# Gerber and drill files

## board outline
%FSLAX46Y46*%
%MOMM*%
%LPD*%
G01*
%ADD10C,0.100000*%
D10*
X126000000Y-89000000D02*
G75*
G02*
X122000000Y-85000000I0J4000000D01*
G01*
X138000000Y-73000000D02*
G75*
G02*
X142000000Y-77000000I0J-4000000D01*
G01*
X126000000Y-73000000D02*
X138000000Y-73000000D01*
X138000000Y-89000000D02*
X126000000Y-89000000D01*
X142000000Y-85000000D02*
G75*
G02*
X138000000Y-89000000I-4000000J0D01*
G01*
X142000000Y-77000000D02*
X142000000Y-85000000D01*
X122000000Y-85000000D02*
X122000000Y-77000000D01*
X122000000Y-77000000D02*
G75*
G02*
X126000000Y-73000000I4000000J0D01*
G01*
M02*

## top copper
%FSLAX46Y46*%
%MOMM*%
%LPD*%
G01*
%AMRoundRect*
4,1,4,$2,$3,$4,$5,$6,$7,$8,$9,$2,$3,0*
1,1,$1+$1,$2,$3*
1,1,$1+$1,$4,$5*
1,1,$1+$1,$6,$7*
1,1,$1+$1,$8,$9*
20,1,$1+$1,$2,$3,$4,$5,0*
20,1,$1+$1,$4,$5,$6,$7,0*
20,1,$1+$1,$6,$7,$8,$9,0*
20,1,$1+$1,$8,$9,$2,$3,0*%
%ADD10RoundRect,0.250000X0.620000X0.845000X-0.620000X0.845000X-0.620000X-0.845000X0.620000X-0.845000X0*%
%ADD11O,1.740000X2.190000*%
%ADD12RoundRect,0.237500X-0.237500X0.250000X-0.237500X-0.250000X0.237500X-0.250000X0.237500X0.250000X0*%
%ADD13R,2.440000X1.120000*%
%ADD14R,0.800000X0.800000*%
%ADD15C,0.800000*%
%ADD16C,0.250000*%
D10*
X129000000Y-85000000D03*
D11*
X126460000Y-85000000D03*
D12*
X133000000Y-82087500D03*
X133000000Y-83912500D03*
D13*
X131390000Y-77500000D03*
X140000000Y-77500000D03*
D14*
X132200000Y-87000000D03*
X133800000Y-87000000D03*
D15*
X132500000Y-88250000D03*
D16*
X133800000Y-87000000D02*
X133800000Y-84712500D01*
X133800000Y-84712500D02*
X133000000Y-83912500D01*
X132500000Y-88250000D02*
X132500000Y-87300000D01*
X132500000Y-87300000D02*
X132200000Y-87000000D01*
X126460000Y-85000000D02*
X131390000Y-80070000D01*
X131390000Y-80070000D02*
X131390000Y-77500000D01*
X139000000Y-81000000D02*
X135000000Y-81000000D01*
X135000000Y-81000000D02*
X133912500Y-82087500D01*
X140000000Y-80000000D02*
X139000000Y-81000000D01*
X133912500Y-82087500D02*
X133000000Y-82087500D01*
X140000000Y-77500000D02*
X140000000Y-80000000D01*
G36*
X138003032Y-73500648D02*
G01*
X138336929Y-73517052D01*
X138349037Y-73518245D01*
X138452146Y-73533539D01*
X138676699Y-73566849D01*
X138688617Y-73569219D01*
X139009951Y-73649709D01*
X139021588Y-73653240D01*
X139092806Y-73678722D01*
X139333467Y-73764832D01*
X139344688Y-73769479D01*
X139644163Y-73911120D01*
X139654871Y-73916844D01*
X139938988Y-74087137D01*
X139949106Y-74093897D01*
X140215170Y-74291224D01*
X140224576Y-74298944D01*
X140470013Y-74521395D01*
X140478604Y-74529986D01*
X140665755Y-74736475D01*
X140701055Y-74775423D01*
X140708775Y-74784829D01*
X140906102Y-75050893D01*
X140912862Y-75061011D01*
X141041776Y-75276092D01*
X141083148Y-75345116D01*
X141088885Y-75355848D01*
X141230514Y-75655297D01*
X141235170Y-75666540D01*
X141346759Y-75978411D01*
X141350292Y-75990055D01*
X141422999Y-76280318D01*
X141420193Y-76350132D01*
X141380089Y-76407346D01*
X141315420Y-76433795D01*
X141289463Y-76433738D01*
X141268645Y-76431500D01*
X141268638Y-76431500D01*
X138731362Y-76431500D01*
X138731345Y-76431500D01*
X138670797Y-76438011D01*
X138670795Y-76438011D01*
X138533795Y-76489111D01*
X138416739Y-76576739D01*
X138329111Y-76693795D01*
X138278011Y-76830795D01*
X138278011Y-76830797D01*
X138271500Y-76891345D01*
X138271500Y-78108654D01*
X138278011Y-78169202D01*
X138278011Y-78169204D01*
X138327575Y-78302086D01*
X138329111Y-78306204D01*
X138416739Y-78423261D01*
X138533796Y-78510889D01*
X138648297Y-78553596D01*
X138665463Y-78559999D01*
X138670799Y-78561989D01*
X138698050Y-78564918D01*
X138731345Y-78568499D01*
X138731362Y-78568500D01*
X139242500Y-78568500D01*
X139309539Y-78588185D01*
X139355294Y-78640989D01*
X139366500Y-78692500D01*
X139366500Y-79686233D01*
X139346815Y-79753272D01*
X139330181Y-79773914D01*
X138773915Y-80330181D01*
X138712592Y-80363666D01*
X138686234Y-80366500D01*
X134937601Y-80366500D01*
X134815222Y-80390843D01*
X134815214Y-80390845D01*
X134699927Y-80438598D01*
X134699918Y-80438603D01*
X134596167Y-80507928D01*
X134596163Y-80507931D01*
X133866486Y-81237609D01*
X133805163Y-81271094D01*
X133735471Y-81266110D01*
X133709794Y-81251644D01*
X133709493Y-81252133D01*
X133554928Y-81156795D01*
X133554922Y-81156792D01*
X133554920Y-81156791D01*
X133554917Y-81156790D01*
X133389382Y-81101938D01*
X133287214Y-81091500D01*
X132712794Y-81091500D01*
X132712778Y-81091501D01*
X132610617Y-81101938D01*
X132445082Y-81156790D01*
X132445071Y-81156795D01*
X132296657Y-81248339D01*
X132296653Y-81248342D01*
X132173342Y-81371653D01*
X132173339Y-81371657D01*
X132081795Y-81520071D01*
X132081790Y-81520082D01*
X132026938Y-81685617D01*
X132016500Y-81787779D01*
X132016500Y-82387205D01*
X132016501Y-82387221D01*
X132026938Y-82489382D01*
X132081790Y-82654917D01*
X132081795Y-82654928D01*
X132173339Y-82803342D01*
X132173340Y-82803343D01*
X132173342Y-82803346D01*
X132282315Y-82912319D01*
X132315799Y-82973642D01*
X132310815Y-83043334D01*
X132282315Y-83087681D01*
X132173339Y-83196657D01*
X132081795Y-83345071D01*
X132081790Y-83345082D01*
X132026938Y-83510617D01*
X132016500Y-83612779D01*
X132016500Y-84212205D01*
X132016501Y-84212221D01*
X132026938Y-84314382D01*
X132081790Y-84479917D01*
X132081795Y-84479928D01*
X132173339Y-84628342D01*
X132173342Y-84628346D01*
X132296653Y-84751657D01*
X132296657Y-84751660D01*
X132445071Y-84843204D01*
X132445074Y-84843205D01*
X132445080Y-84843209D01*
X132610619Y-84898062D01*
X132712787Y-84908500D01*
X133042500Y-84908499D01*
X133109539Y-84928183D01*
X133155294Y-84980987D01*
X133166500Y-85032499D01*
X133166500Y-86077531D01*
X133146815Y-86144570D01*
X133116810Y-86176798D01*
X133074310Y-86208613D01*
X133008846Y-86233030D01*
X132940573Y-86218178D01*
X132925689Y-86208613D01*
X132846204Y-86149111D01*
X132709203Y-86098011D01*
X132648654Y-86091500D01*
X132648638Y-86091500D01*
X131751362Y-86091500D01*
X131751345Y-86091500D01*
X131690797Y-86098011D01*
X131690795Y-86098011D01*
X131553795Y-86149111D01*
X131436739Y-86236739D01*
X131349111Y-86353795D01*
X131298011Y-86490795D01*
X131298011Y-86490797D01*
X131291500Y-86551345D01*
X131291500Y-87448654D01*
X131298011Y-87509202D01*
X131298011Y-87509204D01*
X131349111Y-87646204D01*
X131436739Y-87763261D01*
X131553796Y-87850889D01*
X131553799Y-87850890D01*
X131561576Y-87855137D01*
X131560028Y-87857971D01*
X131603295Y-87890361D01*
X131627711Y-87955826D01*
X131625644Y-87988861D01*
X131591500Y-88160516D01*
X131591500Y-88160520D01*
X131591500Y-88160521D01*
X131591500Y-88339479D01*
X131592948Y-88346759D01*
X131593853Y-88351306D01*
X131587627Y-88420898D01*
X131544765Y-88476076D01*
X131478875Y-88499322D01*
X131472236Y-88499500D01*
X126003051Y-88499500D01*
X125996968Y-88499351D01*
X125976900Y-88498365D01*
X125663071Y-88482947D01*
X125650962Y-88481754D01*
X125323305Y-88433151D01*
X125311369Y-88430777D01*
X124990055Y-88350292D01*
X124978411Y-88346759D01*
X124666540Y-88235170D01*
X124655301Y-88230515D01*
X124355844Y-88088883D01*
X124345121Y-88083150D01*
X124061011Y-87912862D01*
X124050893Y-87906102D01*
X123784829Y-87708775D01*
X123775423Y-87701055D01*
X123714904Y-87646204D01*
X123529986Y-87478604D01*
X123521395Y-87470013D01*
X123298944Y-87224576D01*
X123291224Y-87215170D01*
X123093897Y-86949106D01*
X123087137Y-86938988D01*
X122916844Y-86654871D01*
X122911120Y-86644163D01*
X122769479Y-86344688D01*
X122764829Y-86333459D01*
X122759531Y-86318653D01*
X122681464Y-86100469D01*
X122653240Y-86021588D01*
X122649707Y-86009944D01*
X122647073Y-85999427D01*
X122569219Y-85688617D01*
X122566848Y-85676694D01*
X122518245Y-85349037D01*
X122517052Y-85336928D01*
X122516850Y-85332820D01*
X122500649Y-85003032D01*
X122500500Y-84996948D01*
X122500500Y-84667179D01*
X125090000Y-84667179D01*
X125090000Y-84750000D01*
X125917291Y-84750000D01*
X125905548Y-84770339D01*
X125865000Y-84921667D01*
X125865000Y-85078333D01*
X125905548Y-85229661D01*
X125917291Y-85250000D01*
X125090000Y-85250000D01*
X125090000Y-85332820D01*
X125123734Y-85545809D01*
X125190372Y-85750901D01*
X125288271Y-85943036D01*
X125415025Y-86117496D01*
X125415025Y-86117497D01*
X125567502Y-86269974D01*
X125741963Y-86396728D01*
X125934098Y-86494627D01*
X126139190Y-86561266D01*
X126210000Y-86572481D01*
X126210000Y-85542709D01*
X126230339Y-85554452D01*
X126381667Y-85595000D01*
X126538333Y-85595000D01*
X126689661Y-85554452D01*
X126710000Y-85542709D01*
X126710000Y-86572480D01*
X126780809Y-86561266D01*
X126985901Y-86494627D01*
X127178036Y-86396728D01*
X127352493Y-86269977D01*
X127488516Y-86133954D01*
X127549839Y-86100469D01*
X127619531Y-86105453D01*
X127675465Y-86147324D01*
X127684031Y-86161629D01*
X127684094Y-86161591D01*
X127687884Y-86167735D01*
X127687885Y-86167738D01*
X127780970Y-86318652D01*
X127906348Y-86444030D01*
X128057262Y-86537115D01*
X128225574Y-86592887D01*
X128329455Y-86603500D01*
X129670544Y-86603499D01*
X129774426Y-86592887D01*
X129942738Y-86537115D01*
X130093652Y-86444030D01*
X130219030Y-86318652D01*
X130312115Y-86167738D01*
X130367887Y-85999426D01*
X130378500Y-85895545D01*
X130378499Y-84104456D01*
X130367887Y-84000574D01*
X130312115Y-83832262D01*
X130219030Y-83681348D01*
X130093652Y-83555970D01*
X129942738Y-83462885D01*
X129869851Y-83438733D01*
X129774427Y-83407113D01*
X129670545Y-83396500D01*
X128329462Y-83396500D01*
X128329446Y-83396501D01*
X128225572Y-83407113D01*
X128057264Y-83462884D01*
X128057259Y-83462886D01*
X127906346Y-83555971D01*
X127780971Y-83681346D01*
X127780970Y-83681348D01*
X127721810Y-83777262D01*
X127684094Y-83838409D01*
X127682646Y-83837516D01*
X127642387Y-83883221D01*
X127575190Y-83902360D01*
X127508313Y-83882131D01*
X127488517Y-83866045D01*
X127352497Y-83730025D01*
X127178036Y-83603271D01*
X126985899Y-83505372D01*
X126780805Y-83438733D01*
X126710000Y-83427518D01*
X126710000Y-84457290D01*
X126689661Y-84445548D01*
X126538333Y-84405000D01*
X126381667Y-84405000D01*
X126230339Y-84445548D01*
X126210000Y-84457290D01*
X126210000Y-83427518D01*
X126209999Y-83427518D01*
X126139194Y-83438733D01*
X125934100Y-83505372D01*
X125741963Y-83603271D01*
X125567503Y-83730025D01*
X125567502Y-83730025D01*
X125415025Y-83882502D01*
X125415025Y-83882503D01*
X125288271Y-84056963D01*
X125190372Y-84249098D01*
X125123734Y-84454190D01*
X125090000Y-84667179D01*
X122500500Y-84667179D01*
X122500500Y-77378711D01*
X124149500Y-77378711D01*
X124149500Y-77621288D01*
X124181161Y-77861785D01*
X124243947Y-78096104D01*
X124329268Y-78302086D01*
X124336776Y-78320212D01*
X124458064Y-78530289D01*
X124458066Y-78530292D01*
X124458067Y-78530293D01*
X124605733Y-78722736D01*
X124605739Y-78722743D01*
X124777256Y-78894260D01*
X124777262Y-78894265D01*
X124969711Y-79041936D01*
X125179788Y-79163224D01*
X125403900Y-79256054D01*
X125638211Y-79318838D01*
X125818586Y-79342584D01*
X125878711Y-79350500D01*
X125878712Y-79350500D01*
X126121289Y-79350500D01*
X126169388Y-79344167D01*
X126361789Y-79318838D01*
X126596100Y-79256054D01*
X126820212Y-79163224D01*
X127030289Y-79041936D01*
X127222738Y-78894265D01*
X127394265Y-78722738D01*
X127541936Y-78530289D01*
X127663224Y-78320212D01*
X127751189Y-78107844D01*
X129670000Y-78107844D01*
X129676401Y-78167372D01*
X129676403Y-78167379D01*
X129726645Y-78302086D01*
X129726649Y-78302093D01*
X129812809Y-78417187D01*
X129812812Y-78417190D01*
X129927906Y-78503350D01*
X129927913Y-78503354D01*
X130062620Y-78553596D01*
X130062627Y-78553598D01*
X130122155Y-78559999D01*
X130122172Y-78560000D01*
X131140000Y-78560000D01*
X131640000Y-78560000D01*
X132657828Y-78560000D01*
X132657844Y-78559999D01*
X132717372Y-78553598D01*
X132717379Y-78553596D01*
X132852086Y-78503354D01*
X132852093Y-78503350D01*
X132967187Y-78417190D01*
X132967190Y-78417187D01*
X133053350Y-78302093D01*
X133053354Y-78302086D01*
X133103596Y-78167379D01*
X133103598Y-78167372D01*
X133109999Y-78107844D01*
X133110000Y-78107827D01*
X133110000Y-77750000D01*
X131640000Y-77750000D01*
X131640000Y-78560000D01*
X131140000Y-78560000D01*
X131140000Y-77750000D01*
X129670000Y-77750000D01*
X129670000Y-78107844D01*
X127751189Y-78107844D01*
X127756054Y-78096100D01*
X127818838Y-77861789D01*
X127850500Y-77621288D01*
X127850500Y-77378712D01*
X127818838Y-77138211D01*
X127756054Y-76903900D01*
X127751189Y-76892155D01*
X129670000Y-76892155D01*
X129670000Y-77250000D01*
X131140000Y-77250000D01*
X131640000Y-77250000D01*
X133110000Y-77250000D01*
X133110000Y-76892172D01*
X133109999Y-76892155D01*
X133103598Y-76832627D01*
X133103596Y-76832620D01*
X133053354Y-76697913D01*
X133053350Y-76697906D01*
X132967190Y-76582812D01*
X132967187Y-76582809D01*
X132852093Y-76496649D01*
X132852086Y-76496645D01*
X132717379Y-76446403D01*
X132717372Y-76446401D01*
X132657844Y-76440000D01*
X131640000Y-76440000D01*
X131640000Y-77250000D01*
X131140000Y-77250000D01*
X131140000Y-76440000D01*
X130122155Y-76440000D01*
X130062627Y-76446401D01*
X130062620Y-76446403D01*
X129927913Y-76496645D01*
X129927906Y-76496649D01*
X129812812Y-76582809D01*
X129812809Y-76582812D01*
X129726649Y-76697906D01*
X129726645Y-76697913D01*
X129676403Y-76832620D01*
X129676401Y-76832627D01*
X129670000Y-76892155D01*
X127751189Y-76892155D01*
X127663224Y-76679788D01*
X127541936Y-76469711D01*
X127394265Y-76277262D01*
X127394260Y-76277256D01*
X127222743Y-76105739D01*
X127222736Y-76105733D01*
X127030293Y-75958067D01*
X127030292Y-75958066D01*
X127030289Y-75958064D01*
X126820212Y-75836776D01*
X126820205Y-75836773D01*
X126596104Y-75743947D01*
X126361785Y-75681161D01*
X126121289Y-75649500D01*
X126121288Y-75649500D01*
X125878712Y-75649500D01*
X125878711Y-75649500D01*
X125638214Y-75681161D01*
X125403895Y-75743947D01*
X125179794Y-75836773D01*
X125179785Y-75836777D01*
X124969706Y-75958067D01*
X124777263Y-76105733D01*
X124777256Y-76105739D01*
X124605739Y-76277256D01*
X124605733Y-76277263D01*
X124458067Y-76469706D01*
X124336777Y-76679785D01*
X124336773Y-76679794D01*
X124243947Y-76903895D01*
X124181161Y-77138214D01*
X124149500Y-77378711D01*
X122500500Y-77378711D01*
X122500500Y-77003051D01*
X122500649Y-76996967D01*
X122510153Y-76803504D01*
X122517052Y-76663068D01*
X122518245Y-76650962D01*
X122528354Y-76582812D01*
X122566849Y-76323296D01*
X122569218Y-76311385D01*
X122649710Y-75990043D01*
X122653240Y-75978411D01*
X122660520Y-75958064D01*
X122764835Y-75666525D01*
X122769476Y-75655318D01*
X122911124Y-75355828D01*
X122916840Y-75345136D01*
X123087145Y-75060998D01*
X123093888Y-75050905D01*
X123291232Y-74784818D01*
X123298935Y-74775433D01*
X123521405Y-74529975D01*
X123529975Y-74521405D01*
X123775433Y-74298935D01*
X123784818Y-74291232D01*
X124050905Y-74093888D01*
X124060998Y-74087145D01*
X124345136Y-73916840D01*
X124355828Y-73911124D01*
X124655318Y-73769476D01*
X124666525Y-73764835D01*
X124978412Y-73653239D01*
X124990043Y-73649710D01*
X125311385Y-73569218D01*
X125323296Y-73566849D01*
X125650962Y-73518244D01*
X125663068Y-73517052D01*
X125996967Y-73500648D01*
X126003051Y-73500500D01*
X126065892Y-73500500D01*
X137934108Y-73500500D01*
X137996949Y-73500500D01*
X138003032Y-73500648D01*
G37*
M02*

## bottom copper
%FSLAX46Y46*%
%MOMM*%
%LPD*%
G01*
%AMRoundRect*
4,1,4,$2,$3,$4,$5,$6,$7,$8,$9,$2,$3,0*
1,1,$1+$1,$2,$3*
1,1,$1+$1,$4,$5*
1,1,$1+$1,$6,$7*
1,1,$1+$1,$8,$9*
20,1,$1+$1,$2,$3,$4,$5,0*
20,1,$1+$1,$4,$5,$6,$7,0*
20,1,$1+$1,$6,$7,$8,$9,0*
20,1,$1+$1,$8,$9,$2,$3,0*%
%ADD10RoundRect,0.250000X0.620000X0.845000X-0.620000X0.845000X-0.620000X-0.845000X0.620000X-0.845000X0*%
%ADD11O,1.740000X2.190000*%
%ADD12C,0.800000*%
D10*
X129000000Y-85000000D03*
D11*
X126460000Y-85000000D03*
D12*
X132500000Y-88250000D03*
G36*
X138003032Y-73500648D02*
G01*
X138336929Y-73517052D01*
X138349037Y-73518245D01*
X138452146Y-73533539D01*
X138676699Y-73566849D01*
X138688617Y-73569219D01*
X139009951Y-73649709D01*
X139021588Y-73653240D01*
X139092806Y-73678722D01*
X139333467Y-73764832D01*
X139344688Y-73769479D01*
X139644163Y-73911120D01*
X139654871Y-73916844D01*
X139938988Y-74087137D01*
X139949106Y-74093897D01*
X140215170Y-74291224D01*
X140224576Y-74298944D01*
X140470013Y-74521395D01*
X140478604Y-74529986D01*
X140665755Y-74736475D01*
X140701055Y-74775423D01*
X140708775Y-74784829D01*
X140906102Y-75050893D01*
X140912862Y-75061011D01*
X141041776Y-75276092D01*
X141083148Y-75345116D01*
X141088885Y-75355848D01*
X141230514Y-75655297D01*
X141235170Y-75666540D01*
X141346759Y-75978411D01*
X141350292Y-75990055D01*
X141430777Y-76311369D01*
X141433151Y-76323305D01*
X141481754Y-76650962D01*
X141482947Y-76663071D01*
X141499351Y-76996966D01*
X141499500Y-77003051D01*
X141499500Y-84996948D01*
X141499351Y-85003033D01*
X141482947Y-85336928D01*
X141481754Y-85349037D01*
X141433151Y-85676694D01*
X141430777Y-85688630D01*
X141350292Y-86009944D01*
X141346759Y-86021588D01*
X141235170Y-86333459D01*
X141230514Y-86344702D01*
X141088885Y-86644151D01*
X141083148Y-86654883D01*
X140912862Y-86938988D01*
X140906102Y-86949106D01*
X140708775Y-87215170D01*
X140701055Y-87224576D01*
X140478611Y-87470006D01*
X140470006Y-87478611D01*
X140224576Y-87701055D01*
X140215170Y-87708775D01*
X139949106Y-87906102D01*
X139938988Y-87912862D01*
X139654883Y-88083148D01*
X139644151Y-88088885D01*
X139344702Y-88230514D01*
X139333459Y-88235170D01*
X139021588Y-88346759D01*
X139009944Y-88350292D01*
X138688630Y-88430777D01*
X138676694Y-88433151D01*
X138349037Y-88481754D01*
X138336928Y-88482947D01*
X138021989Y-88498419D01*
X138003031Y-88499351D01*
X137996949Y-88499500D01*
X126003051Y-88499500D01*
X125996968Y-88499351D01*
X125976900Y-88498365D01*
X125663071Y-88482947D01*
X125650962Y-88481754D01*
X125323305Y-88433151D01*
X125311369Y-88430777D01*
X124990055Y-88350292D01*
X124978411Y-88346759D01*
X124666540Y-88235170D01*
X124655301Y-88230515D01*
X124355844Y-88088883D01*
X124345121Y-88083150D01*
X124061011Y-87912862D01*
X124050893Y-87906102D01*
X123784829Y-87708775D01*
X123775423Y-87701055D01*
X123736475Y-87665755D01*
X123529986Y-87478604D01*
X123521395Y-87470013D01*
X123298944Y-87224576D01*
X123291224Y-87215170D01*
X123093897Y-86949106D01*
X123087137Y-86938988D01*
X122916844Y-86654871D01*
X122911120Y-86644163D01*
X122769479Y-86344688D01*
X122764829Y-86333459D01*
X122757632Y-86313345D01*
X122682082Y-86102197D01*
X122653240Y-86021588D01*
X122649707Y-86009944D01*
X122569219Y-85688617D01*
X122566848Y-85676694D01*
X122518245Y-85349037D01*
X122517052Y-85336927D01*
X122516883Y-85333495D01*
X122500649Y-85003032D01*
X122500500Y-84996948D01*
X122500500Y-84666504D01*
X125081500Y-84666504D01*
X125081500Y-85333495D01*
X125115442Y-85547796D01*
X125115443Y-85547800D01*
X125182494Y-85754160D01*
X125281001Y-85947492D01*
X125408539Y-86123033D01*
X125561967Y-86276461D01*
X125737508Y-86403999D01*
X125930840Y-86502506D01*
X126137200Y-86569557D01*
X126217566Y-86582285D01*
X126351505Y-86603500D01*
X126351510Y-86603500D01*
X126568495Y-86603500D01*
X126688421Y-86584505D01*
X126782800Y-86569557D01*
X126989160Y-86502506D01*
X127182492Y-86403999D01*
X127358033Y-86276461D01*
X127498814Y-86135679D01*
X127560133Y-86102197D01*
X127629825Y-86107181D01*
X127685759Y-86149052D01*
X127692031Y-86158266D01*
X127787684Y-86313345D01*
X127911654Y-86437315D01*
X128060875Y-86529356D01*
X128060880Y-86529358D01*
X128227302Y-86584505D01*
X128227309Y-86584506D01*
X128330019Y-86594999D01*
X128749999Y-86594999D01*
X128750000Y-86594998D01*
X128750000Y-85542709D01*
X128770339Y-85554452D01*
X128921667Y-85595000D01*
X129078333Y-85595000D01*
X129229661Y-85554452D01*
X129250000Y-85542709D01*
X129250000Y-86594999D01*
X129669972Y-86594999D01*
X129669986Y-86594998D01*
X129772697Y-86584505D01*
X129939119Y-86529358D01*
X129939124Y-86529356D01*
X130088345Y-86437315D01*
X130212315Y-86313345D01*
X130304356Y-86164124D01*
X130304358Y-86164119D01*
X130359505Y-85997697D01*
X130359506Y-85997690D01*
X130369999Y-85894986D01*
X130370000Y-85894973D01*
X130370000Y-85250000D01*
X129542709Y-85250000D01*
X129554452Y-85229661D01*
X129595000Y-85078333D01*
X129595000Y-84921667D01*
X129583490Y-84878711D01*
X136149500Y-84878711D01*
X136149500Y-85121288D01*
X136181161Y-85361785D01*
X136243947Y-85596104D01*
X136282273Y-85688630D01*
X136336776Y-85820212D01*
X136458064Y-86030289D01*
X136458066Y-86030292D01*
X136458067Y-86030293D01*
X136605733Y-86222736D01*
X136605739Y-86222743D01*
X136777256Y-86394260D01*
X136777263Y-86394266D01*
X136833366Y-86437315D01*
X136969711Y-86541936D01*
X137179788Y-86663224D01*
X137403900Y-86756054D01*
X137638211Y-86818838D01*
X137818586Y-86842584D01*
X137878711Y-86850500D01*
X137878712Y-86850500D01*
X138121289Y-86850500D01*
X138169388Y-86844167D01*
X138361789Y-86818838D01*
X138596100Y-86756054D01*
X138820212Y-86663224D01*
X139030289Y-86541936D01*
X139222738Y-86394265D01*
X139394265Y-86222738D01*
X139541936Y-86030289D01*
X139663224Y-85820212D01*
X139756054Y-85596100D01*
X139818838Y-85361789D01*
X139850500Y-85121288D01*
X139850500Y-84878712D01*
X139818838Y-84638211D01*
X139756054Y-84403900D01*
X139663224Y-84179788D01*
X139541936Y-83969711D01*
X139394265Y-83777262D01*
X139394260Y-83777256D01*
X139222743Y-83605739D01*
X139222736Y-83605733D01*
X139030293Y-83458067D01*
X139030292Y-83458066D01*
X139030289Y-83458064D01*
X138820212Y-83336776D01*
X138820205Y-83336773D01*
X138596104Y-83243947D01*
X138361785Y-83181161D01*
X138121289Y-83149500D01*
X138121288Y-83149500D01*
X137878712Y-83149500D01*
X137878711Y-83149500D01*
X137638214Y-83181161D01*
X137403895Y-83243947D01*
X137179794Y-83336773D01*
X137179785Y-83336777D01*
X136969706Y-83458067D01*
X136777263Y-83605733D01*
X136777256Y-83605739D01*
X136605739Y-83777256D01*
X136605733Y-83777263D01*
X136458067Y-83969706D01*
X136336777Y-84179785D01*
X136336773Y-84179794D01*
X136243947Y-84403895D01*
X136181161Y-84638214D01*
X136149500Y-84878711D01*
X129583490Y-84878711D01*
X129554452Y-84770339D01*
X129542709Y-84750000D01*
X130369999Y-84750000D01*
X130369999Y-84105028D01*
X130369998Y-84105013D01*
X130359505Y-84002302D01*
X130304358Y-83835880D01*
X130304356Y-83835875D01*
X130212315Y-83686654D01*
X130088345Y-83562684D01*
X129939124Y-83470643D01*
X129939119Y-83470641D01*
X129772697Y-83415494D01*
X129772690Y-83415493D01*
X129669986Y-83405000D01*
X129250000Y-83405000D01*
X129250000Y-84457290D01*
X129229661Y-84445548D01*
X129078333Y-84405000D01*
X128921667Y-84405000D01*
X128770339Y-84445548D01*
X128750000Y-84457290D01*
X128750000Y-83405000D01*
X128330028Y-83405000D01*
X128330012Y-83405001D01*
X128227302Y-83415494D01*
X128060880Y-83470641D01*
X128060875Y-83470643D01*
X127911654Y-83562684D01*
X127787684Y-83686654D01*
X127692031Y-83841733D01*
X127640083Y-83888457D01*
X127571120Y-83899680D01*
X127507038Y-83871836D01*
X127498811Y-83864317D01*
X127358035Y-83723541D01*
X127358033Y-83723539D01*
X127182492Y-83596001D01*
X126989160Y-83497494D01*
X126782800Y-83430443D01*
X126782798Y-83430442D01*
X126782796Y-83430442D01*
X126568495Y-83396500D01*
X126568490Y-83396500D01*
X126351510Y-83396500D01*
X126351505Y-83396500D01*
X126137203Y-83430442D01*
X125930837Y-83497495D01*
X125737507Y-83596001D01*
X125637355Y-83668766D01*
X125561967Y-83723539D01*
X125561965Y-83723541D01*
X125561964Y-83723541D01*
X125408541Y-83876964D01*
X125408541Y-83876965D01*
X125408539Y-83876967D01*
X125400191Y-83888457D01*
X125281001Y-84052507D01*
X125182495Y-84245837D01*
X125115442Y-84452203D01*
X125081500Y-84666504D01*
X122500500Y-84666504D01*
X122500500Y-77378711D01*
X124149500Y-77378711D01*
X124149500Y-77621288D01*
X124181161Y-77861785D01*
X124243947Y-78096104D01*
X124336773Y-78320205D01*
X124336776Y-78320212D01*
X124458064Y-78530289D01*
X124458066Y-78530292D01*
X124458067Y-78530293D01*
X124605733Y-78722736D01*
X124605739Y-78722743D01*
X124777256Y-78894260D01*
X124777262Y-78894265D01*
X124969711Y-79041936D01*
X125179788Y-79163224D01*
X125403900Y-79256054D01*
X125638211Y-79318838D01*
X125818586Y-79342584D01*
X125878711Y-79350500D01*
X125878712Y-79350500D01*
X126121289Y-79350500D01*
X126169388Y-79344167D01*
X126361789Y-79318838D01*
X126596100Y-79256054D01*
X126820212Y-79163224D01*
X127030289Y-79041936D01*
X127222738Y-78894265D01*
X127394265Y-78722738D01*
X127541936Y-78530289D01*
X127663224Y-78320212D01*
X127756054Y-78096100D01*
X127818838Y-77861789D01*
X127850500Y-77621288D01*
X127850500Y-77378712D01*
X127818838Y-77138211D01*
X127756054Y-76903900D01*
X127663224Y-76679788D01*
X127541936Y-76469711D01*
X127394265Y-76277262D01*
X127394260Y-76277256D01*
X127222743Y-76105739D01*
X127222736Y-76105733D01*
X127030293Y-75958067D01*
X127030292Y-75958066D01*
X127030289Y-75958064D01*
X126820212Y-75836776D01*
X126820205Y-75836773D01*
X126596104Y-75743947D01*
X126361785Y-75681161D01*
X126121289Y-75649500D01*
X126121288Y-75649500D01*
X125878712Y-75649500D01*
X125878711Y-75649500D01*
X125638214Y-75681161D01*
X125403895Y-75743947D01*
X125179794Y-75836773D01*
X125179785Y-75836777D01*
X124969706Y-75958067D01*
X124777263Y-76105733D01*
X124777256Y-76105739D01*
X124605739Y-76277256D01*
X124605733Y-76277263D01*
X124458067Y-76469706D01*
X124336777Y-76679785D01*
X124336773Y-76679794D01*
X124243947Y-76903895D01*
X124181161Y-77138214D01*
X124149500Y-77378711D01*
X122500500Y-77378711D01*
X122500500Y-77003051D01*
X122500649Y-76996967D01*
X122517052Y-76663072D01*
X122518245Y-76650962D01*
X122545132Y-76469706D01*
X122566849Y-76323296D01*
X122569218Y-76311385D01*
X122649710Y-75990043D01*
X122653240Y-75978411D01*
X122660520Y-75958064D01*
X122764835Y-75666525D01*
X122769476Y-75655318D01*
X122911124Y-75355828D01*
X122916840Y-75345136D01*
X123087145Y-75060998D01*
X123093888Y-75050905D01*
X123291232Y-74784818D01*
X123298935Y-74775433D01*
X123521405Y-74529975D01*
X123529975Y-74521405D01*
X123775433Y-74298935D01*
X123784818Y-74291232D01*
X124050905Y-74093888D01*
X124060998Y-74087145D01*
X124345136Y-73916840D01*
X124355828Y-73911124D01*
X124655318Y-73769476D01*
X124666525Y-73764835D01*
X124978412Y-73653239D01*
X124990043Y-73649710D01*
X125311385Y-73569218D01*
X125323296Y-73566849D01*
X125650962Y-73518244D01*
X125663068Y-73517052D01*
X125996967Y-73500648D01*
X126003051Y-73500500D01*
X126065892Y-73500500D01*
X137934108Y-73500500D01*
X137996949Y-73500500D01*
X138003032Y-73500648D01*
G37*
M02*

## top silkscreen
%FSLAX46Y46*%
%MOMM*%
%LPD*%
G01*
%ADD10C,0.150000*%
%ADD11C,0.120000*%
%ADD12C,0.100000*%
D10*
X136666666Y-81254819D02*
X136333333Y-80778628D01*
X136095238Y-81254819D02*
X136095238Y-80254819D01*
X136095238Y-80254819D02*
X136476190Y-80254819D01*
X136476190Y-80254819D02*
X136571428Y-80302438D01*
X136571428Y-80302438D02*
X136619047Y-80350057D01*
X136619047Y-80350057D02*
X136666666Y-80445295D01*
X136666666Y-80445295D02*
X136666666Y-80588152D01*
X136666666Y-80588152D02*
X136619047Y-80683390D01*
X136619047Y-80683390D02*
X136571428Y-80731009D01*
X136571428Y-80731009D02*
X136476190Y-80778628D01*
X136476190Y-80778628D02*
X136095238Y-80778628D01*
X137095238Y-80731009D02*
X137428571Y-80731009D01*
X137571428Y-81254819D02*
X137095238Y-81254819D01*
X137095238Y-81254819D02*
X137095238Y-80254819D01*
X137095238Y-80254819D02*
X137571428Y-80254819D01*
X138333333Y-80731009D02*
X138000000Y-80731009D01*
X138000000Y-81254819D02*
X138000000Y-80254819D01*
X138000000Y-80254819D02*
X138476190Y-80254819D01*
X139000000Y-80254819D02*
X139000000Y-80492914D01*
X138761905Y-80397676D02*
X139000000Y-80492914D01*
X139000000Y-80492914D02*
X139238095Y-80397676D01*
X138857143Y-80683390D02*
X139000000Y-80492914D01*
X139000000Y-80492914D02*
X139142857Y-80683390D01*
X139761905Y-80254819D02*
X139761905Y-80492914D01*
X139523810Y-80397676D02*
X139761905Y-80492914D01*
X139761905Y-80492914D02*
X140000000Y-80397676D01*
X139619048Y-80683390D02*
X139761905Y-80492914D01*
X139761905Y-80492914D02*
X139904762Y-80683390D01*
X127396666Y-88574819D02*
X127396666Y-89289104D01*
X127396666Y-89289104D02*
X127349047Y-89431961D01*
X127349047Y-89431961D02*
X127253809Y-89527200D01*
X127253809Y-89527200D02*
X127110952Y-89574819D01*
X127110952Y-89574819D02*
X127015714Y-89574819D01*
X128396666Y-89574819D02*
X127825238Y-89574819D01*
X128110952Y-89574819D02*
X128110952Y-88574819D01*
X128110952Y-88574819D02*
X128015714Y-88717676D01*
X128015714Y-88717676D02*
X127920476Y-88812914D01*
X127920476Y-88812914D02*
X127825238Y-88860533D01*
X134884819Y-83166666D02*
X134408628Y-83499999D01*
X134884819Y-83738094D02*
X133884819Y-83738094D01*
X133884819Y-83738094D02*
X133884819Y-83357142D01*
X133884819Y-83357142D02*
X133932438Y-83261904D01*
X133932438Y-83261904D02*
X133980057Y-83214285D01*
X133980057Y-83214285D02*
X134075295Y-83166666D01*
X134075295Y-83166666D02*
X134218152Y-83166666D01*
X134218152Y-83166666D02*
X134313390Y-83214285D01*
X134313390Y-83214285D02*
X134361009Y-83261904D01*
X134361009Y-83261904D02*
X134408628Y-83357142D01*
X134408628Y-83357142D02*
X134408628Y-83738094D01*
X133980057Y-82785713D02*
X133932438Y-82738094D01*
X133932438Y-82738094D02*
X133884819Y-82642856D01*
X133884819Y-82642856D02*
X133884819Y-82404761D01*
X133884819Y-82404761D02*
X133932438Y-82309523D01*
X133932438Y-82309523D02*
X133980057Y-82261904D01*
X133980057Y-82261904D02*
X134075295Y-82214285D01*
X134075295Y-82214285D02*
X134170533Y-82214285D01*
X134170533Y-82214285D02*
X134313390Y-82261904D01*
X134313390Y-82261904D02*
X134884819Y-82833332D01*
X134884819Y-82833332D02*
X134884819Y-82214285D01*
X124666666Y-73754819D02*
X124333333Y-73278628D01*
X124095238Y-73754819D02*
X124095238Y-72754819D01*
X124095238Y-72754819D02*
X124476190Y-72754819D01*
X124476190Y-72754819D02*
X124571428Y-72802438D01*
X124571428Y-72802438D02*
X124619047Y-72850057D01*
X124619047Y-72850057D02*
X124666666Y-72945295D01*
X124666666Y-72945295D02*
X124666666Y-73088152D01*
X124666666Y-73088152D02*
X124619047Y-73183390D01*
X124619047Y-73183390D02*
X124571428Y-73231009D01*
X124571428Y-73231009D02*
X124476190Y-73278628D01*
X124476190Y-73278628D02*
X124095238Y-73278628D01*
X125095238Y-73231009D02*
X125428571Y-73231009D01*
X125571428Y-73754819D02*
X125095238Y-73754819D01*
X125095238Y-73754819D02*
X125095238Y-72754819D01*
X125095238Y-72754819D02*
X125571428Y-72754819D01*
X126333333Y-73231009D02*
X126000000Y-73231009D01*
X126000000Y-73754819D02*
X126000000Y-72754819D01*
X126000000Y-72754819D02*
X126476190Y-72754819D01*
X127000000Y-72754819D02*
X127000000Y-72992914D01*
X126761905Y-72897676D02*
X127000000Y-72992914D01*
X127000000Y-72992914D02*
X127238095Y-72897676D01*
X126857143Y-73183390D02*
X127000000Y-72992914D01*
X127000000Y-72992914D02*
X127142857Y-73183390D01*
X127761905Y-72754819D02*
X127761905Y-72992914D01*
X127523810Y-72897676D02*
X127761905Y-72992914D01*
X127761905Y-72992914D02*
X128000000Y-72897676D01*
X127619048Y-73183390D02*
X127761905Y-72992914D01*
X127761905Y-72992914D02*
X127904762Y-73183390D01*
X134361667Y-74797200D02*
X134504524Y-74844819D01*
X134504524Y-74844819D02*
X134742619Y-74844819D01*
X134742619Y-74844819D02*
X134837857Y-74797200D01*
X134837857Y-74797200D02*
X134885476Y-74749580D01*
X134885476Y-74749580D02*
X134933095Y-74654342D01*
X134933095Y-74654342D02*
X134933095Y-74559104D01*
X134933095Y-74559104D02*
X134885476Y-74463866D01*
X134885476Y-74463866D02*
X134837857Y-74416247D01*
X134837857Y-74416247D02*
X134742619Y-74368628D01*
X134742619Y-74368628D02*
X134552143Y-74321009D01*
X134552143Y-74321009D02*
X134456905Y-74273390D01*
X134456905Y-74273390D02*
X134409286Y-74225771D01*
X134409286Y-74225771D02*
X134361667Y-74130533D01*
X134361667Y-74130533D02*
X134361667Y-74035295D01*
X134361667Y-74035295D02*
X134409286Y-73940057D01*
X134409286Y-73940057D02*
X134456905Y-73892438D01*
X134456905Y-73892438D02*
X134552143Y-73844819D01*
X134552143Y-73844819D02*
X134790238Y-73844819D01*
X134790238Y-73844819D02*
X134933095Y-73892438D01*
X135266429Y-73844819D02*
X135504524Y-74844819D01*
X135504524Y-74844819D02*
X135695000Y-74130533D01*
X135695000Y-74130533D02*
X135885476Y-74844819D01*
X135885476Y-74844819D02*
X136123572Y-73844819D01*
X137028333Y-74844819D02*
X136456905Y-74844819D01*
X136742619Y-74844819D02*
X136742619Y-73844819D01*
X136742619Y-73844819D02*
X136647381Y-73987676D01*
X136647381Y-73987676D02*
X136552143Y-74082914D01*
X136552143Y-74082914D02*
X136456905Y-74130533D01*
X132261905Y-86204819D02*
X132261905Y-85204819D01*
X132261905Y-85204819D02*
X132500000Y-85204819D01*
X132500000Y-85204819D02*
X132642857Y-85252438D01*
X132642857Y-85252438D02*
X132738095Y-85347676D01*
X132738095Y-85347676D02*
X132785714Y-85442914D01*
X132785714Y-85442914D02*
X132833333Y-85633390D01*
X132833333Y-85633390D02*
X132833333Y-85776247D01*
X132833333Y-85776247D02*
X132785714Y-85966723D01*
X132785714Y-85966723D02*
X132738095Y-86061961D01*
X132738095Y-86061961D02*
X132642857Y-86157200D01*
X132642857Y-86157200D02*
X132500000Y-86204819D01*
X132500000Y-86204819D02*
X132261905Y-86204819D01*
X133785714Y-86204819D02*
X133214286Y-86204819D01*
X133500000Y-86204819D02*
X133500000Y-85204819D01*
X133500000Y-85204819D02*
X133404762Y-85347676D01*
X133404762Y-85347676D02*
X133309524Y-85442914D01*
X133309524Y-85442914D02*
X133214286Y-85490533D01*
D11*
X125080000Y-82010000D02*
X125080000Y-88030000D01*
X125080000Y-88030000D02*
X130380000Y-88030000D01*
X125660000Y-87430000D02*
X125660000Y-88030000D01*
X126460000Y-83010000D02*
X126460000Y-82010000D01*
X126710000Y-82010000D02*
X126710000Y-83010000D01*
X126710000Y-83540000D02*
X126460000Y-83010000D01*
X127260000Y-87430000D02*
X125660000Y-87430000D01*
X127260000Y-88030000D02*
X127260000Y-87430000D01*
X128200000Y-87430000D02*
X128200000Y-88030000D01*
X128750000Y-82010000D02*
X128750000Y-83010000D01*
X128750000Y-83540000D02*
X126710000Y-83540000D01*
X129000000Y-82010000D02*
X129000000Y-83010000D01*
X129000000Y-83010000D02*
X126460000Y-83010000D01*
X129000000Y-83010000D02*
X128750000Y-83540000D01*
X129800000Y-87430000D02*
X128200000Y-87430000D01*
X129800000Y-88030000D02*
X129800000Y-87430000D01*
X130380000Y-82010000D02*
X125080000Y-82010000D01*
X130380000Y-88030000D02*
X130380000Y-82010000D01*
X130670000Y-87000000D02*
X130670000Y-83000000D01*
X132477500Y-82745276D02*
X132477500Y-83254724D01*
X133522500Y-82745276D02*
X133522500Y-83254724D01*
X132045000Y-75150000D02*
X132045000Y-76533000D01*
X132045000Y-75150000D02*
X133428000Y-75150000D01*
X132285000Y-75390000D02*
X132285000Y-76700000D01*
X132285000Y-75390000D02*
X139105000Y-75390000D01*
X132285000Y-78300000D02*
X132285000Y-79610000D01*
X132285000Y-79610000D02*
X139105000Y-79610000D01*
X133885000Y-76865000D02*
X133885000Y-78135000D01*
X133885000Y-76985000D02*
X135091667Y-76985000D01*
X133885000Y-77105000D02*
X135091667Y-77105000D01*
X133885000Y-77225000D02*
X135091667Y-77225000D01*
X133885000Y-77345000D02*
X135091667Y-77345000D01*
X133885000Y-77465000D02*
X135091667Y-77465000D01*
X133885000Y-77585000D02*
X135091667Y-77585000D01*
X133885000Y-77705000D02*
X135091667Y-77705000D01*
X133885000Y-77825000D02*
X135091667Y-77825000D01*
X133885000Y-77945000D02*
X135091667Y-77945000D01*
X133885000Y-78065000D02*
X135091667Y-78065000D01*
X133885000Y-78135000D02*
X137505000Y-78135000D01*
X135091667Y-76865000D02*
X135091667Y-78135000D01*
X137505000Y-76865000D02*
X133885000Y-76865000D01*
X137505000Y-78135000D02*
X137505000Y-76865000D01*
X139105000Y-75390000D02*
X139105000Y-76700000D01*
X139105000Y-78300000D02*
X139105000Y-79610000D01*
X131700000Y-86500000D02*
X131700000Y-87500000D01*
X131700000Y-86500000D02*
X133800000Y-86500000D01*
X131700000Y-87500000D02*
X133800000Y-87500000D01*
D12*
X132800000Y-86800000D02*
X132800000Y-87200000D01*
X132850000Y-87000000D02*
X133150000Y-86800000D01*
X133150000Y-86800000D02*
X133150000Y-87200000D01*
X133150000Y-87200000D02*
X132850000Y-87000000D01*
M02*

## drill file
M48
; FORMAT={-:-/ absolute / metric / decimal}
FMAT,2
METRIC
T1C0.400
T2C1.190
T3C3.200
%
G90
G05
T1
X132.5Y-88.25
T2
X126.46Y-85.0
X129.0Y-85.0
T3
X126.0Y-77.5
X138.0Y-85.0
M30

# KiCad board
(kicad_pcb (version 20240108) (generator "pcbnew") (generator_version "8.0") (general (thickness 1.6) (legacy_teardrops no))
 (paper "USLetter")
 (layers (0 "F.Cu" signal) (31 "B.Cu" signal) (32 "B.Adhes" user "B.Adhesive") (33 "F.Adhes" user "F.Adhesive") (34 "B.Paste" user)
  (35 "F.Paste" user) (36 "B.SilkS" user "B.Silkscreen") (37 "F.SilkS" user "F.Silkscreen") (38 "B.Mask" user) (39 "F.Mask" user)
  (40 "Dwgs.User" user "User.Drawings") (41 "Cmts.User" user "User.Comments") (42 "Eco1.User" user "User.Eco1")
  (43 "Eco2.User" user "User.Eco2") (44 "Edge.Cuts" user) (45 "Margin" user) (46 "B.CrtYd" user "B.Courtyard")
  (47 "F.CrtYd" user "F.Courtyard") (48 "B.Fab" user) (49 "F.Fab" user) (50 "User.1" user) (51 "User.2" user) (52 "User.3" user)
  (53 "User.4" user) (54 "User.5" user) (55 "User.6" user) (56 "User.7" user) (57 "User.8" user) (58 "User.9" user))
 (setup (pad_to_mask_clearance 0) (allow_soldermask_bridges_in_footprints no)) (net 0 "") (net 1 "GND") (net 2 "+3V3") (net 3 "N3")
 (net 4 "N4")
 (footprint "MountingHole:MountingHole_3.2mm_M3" (layer "F.Cu") (at 138 85)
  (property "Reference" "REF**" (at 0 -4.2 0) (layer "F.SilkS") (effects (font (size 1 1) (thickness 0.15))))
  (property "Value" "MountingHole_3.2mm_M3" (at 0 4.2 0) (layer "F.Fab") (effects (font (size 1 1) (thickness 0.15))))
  (pad "" np_thru_hole circle (at 0 0) (size 3.2 3.2) (drill 3.2) (layers "*.Cu" "*.Mask")))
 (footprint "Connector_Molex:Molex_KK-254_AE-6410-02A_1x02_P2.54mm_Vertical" (layer "F.Cu") (at 129 85 180)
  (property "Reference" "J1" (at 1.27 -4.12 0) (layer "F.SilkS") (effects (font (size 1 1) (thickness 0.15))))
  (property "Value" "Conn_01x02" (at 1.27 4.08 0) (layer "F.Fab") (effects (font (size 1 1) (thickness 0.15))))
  (fp_line (start 3.92 2.99) (end 3.92 -3.03) (stroke (width 0.12) (type solid)) (layer "F.SilkS"))
  (fp_line (start 3.92 -3.03) (end -1.38 -3.03) (stroke (width 0.12) (type solid)) (layer "F.SilkS"))
  (fp_line (start 3.34 -2.43) (end 3.34 -3.03) (stroke (width 0.12) (type solid)) (layer "F.SilkS"))
  (fp_line (start 2.54 1.99) (end 2.54 2.99) (stroke (width 0.12) (type solid)) (layer "F.SilkS"))
  (fp_line (start 2.29 2.99) (end 2.29 1.99) (stroke (width 0.12) (type solid)) (layer "F.SilkS"))
  (fp_line (start 2.29 1.46) (end 2.54 1.99) (stroke (width 0.12) (type solid)) (layer "F.SilkS"))
  (fp_line (start 1.74 -2.43) (end 3.34 -2.43) (stroke (width 0.12) (type solid)) (layer "F.SilkS"))
  (fp_line (start 1.74 -3.03) (end 1.74 -2.43) (stroke (width 0.12) (type solid)) (layer "F.SilkS"))
  (fp_line (start 0.8 -2.43) (end 0.8 -3.03) (stroke (width 0.12) (type solid)) (layer "F.SilkS"))
  (fp_line (start 0.25 2.99) (end 0.25 1.99) (stroke (width 0.12) (type solid)) (layer "F.SilkS"))
  (fp_line (start 0.25 1.46) (end 2.29 1.46) (stroke (width 0.12) (type solid)) (layer "F.SilkS"))
  (fp_line (start 0 2.99) (end 0 1.99) (stroke (width 0.12) (type solid)) (layer "F.SilkS"))
  (fp_line (start 0 1.99) (end 2.54 1.99) (stroke (width 0.12) (type solid)) (layer "F.SilkS"))
  (fp_line (start 0 1.99) (end 0.25 1.46) (stroke (width 0.12) (type solid)) (layer "F.SilkS"))
  (fp_line (start -0.8 -2.43) (end 0.8 -2.43) (stroke (width 0.12) (type solid)) (layer "F.SilkS"))
  (fp_line (start -0.8 -3.03) (end -0.8 -2.43) (stroke (width 0.12) (type solid)) (layer "F.SilkS"))
  (fp_line (start -1.38 2.99) (end 3.92 2.99) (stroke (width 0.12) (type solid)) (layer "F.SilkS"))
  (fp_line (start -1.38 -3.03) (end -1.38 2.99) (stroke (width 0.12) (type solid)) (layer "F.SilkS"))
  (fp_line (start -1.67 -2) (end -1.67 2) (stroke (width 0.12) (type solid)) (layer "F.SilkS"))
  (pad "1" thru_hole roundrect (at 0 0 180) (size 1.74 2.19) (drill 1.19) (layers "*.Cu" "*.Mask") (remove_unused_layers no)
   (roundrect_rratio 0.143678) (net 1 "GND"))
  (pad "2" thru_hole oval (at 2.54 0 180) (size 1.74 2.19) (drill 1.19) (layers "*.Cu" "*.Mask") (remove_unused_layers no) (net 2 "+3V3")))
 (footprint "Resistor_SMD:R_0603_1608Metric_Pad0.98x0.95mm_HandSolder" (layer "F.Cu") (at 133 83 -90)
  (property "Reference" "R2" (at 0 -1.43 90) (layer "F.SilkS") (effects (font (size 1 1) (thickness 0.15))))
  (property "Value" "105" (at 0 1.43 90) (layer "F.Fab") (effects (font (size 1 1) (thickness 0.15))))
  (fp_line (start -0.254724 0.5225) (end 0.254724 0.5225) (stroke (width 0.12) (type solid)) (layer "F.SilkS"))
  (fp_line (start -0.254724 -0.5225) (end 0.254724 -0.5225) (stroke (width 0.12) (type solid)) (layer "F.SilkS"))
  (pad "1" smd roundrect (at -0.9125 0 270) (size 0.975 0.95) (layers "F.Cu" "F.Paste" "F.Mask") (roundrect_rratio 0.25) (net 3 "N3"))
  (pad "2" smd roundrect (at 0.9125 0 270) (size 0.975 0.95) (layers "F.Cu" "F.Paste" "F.Mask") (roundrect_rratio 0.25) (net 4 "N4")))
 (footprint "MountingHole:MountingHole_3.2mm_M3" (layer "F.Cu") (at 126 77.5)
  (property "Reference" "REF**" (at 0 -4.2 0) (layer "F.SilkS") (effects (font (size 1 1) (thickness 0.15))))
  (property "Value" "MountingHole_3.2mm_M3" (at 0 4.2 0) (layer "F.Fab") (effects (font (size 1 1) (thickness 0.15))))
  (pad "" np_thru_hole circle (at 0 0) (size 3.2 3.2) (drill 3.2) (layers "*.Cu" "*.Mask")))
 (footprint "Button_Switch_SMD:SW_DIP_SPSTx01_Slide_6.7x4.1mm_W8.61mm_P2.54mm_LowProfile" (layer "F.Cu") (at 135.695 77.5)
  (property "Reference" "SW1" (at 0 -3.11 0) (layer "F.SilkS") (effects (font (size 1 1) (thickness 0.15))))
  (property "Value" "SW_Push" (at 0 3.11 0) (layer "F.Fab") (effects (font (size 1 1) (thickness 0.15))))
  (fp_line (start -3.65 -2.35) (end -3.65 -0.967) (stroke (width 0.12) (type solid)) (layer "F.SilkS"))
  (fp_line (start -3.65 -2.35) (end -2.267 -2.35) (stroke (width 0.12) (type solid)) (layer "F.SilkS"))
  (fp_line (start -3.41 -2.11) (end -3.41 -0.8) (stroke (width 0.12) (type solid)) (layer "F.SilkS"))
  (fp_line (start -3.41 -2.11) (end 3.41 -2.11) (stroke (width 0.12) (type solid)) (layer "F.SilkS"))
  (fp_line (start -3.41 0.8) (end -3.41 2.11) (stroke (width 0.12) (type solid)) (layer "F.SilkS"))
  (fp_line (start -3.41 2.11) (end 3.41 2.11) (stroke (width 0.12) (type solid)) (layer "F.SilkS"))
  (fp_line (start -1.81 -0.635) (end -1.81 0.635) (stroke (width 0.12) (type solid)) (layer "F.SilkS"))
  (fp_line (start -1.81 -0.515) (end -0.603333 -0.515) (stroke (width 0.12) (type solid)) (layer "F.SilkS"))
  (fp_line (start -1.81 -0.395) (end -0.603333 -0.395) (stroke (width 0.12) (type solid)) (layer "F.SilkS"))
  (fp_line (start -1.81 -0.275) (end -0.603333 -0.275) (stroke (width 0.12) (type solid)) (layer "F.SilkS"))
  (fp_line (start -1.81 -0.155) (end -0.603333 -0.155) (stroke (width 0.12) (type solid)) (layer "F.SilkS"))
  (fp_line (start -1.81 -0.035) (end -0.603333 -0.035) (stroke (width 0.12) (type solid)) (layer "F.SilkS"))
  (fp_line (start -1.81 0.085) (end -0.603333 0.085) (stroke (width 0.12) (type solid)) (layer "F.SilkS"))
  (fp_line (start -1.81 0.205) (end -0.603333 0.205) (stroke (width 0.12) (type solid)) (layer "F.SilkS"))
  (fp_line (start -1.81 0.325) (end -0.603333 0.325) (stroke (width 0.12) (type solid)) (layer "F.SilkS"))
  (fp_line (start -1.81 0.445) (end -0.603333 0.445) (stroke (width 0.12) (type solid)) (layer "F.SilkS"))
  (fp_line (start -1.81 0.565) (end -0.603333 0.565) (stroke (width 0.12) (type solid)) (layer "F.SilkS"))
  (fp_line (start -1.81 0.635) (end 1.81 0.635) (stroke (width 0.12) (type solid)) (layer "F.SilkS"))
  (fp_line (start -0.603333 -0.635) (end -0.603333 0.635) (stroke (width 0.12) (type solid)) (layer "F.SilkS"))
  (fp_line (start 1.81 -0.635) (end -1.81 -0.635) (stroke (width 0.12) (type solid)) (layer "F.SilkS"))
  (fp_line (start 1.81 0.635) (end 1.81 -0.635) (stroke (width 0.12) (type solid)) (layer "F.SilkS"))
  (fp_line (start 3.41 -2.11) (end 3.41 -0.8) (stroke (width 0.12) (type solid)) (layer "F.SilkS"))
  (fp_line (start 3.41 0.8) (end 3.41 2.11) (stroke (width 0.12) (type solid)) (layer "F.SilkS"))
  (pad "1" smd rect (at -4.305 0) (size 2.44 1.12) (layers "F.Cu" "F.Paste" "F.Mask") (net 2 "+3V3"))
  (pad "2" smd rect (at 4.305 0) (size 2.44 1.12) (layers "F.Cu" "F.Paste" "F.Mask") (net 3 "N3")))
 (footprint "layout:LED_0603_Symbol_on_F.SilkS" (layer "F.Cu") (at 133 87)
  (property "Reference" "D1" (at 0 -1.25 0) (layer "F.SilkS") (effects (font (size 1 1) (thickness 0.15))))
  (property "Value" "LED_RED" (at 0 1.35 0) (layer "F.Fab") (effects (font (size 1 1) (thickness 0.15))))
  (fp_line (start -1.3 -0.5) (end -1.3 0.5) (stroke (width 0.12) (type solid)) (layer "F.SilkS"))
  (fp_line (start -1.3 -0.5) (end 0.8 -0.5) (stroke (width 0.12) (type solid)) (layer "F.SilkS"))
  (fp_line (start -1.3 0.5) (end 0.8 0.5) (stroke (width 0.12) (type solid)) (layer "F.SilkS"))
  (fp_line (start -0.2 -0.2) (end -0.2 0.2) (stroke (width 0.1) (type solid)) (layer "F.SilkS"))
  (fp_line (start -0.15 0) (end 0.15 -0.2) (stroke (width 0.1) (type solid)) (layer "F.SilkS"))
  (fp_line (start 0.15 -0.2) (end 0.15 0.2) (stroke (width 0.1) (type solid)) (layer "F.SilkS"))
  (fp_line (start 0.15 0.2) (end -0.15 0) (stroke (width 0.1) (type solid)) (layer "F.SilkS"))
  (pad "1" smd rect (at -0.8 0 180) (size 0.8 0.8) (layers "F.Cu" "F.Paste" "F.Mask") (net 1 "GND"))
  (pad "2" smd rect (at 0.8 0 180) (size 0.8 0.8) (layers "F.Cu" "F.Paste" "F.Mask") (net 4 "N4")))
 (gr_arc (start 126 89) (mid 123.171573 87.828427) (end 122 85) (stroke (width 0.1) (type default)) (layer "Edge.Cuts"))
 (gr_arc (start 138 73) (mid 140.828427 74.171573) (end 142 77) (stroke (width 0.1) (type default)) (layer "Edge.Cuts"))
 (gr_line (start 126 73) (end 138 73) (stroke (width 0.1) (type default)) (layer "Edge.Cuts"))
 (gr_line (start 138 89) (end 126 89) (stroke (width 0.1) (type default)) (layer "Edge.Cuts"))
 (gr_arc (start 142 85) (mid 140.828427 87.828427) (end 138 89) (stroke (width 0.1) (type default)) (layer "Edge.Cuts"))
 (gr_line (start 142 77) (end 142 85) (stroke (width 0.1) (type default)) (layer "Edge.Cuts"))
 (gr_line (start 122 85) (end 122 77) (stroke (width 0.1) (type default)) (layer "Edge.Cuts"))
 (gr_arc (start 122 77) (mid 123.171573 74.171573) (end 126 73) (stroke (width 0.1) (type default)) (layer "Edge.Cuts"))
 (segment (start 133.8 87) (end 133.8 84.7125) (width 0.25) (layer "F.Cu") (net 4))
 (segment (start 133.8 84.7125) (end 133 83.9125) (width 0.25) (layer "F.Cu") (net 4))
 (segment (start 132.5 88.25) (end 132.5 87.3) (width 0.25) (layer "F.Cu") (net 1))
 (segment (start 132.5 87.3) (end 132.2 87) (width 0.25) (layer "F.Cu") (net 1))
 (via (at 132.5 88.25) (size 0.8) (drill 0.4) (layers "F.Cu" "B.Cu") (free yes) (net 1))
 (segment (start 126.46 85) (end 131.39 80.07) (width 0.25) (layer "F.Cu") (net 2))
 (segment (start 131.39 80.07) (end 131.39 77.5) (width 0.25) (layer "F.Cu") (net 2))
 (segment (start 139 81) (end 135 81) (width 0.25) (layer "F.Cu") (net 3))
 (segment (start 135 81) (end 133.9125 82.0875) (width 0.25) (layer "F.Cu") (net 3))
 (segment (start 140 80) (end 139 81) (width 0.25) (layer "F.Cu") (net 3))
 (segment (start 133.9125 82.0875) (end 133 82.0875) (width 0.25) (layer "F.Cu") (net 3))
 (segment (start 140 77.5) (end 140 80) (width 0.25) (layer "F.Cu") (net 3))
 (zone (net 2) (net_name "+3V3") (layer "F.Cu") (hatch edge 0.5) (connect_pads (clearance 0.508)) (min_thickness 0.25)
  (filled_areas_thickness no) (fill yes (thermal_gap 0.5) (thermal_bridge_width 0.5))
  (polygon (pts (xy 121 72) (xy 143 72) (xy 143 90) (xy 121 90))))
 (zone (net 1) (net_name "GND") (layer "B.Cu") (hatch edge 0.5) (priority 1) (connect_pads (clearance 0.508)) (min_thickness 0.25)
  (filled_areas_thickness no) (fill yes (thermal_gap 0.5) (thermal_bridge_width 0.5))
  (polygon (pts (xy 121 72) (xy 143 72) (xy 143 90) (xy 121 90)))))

